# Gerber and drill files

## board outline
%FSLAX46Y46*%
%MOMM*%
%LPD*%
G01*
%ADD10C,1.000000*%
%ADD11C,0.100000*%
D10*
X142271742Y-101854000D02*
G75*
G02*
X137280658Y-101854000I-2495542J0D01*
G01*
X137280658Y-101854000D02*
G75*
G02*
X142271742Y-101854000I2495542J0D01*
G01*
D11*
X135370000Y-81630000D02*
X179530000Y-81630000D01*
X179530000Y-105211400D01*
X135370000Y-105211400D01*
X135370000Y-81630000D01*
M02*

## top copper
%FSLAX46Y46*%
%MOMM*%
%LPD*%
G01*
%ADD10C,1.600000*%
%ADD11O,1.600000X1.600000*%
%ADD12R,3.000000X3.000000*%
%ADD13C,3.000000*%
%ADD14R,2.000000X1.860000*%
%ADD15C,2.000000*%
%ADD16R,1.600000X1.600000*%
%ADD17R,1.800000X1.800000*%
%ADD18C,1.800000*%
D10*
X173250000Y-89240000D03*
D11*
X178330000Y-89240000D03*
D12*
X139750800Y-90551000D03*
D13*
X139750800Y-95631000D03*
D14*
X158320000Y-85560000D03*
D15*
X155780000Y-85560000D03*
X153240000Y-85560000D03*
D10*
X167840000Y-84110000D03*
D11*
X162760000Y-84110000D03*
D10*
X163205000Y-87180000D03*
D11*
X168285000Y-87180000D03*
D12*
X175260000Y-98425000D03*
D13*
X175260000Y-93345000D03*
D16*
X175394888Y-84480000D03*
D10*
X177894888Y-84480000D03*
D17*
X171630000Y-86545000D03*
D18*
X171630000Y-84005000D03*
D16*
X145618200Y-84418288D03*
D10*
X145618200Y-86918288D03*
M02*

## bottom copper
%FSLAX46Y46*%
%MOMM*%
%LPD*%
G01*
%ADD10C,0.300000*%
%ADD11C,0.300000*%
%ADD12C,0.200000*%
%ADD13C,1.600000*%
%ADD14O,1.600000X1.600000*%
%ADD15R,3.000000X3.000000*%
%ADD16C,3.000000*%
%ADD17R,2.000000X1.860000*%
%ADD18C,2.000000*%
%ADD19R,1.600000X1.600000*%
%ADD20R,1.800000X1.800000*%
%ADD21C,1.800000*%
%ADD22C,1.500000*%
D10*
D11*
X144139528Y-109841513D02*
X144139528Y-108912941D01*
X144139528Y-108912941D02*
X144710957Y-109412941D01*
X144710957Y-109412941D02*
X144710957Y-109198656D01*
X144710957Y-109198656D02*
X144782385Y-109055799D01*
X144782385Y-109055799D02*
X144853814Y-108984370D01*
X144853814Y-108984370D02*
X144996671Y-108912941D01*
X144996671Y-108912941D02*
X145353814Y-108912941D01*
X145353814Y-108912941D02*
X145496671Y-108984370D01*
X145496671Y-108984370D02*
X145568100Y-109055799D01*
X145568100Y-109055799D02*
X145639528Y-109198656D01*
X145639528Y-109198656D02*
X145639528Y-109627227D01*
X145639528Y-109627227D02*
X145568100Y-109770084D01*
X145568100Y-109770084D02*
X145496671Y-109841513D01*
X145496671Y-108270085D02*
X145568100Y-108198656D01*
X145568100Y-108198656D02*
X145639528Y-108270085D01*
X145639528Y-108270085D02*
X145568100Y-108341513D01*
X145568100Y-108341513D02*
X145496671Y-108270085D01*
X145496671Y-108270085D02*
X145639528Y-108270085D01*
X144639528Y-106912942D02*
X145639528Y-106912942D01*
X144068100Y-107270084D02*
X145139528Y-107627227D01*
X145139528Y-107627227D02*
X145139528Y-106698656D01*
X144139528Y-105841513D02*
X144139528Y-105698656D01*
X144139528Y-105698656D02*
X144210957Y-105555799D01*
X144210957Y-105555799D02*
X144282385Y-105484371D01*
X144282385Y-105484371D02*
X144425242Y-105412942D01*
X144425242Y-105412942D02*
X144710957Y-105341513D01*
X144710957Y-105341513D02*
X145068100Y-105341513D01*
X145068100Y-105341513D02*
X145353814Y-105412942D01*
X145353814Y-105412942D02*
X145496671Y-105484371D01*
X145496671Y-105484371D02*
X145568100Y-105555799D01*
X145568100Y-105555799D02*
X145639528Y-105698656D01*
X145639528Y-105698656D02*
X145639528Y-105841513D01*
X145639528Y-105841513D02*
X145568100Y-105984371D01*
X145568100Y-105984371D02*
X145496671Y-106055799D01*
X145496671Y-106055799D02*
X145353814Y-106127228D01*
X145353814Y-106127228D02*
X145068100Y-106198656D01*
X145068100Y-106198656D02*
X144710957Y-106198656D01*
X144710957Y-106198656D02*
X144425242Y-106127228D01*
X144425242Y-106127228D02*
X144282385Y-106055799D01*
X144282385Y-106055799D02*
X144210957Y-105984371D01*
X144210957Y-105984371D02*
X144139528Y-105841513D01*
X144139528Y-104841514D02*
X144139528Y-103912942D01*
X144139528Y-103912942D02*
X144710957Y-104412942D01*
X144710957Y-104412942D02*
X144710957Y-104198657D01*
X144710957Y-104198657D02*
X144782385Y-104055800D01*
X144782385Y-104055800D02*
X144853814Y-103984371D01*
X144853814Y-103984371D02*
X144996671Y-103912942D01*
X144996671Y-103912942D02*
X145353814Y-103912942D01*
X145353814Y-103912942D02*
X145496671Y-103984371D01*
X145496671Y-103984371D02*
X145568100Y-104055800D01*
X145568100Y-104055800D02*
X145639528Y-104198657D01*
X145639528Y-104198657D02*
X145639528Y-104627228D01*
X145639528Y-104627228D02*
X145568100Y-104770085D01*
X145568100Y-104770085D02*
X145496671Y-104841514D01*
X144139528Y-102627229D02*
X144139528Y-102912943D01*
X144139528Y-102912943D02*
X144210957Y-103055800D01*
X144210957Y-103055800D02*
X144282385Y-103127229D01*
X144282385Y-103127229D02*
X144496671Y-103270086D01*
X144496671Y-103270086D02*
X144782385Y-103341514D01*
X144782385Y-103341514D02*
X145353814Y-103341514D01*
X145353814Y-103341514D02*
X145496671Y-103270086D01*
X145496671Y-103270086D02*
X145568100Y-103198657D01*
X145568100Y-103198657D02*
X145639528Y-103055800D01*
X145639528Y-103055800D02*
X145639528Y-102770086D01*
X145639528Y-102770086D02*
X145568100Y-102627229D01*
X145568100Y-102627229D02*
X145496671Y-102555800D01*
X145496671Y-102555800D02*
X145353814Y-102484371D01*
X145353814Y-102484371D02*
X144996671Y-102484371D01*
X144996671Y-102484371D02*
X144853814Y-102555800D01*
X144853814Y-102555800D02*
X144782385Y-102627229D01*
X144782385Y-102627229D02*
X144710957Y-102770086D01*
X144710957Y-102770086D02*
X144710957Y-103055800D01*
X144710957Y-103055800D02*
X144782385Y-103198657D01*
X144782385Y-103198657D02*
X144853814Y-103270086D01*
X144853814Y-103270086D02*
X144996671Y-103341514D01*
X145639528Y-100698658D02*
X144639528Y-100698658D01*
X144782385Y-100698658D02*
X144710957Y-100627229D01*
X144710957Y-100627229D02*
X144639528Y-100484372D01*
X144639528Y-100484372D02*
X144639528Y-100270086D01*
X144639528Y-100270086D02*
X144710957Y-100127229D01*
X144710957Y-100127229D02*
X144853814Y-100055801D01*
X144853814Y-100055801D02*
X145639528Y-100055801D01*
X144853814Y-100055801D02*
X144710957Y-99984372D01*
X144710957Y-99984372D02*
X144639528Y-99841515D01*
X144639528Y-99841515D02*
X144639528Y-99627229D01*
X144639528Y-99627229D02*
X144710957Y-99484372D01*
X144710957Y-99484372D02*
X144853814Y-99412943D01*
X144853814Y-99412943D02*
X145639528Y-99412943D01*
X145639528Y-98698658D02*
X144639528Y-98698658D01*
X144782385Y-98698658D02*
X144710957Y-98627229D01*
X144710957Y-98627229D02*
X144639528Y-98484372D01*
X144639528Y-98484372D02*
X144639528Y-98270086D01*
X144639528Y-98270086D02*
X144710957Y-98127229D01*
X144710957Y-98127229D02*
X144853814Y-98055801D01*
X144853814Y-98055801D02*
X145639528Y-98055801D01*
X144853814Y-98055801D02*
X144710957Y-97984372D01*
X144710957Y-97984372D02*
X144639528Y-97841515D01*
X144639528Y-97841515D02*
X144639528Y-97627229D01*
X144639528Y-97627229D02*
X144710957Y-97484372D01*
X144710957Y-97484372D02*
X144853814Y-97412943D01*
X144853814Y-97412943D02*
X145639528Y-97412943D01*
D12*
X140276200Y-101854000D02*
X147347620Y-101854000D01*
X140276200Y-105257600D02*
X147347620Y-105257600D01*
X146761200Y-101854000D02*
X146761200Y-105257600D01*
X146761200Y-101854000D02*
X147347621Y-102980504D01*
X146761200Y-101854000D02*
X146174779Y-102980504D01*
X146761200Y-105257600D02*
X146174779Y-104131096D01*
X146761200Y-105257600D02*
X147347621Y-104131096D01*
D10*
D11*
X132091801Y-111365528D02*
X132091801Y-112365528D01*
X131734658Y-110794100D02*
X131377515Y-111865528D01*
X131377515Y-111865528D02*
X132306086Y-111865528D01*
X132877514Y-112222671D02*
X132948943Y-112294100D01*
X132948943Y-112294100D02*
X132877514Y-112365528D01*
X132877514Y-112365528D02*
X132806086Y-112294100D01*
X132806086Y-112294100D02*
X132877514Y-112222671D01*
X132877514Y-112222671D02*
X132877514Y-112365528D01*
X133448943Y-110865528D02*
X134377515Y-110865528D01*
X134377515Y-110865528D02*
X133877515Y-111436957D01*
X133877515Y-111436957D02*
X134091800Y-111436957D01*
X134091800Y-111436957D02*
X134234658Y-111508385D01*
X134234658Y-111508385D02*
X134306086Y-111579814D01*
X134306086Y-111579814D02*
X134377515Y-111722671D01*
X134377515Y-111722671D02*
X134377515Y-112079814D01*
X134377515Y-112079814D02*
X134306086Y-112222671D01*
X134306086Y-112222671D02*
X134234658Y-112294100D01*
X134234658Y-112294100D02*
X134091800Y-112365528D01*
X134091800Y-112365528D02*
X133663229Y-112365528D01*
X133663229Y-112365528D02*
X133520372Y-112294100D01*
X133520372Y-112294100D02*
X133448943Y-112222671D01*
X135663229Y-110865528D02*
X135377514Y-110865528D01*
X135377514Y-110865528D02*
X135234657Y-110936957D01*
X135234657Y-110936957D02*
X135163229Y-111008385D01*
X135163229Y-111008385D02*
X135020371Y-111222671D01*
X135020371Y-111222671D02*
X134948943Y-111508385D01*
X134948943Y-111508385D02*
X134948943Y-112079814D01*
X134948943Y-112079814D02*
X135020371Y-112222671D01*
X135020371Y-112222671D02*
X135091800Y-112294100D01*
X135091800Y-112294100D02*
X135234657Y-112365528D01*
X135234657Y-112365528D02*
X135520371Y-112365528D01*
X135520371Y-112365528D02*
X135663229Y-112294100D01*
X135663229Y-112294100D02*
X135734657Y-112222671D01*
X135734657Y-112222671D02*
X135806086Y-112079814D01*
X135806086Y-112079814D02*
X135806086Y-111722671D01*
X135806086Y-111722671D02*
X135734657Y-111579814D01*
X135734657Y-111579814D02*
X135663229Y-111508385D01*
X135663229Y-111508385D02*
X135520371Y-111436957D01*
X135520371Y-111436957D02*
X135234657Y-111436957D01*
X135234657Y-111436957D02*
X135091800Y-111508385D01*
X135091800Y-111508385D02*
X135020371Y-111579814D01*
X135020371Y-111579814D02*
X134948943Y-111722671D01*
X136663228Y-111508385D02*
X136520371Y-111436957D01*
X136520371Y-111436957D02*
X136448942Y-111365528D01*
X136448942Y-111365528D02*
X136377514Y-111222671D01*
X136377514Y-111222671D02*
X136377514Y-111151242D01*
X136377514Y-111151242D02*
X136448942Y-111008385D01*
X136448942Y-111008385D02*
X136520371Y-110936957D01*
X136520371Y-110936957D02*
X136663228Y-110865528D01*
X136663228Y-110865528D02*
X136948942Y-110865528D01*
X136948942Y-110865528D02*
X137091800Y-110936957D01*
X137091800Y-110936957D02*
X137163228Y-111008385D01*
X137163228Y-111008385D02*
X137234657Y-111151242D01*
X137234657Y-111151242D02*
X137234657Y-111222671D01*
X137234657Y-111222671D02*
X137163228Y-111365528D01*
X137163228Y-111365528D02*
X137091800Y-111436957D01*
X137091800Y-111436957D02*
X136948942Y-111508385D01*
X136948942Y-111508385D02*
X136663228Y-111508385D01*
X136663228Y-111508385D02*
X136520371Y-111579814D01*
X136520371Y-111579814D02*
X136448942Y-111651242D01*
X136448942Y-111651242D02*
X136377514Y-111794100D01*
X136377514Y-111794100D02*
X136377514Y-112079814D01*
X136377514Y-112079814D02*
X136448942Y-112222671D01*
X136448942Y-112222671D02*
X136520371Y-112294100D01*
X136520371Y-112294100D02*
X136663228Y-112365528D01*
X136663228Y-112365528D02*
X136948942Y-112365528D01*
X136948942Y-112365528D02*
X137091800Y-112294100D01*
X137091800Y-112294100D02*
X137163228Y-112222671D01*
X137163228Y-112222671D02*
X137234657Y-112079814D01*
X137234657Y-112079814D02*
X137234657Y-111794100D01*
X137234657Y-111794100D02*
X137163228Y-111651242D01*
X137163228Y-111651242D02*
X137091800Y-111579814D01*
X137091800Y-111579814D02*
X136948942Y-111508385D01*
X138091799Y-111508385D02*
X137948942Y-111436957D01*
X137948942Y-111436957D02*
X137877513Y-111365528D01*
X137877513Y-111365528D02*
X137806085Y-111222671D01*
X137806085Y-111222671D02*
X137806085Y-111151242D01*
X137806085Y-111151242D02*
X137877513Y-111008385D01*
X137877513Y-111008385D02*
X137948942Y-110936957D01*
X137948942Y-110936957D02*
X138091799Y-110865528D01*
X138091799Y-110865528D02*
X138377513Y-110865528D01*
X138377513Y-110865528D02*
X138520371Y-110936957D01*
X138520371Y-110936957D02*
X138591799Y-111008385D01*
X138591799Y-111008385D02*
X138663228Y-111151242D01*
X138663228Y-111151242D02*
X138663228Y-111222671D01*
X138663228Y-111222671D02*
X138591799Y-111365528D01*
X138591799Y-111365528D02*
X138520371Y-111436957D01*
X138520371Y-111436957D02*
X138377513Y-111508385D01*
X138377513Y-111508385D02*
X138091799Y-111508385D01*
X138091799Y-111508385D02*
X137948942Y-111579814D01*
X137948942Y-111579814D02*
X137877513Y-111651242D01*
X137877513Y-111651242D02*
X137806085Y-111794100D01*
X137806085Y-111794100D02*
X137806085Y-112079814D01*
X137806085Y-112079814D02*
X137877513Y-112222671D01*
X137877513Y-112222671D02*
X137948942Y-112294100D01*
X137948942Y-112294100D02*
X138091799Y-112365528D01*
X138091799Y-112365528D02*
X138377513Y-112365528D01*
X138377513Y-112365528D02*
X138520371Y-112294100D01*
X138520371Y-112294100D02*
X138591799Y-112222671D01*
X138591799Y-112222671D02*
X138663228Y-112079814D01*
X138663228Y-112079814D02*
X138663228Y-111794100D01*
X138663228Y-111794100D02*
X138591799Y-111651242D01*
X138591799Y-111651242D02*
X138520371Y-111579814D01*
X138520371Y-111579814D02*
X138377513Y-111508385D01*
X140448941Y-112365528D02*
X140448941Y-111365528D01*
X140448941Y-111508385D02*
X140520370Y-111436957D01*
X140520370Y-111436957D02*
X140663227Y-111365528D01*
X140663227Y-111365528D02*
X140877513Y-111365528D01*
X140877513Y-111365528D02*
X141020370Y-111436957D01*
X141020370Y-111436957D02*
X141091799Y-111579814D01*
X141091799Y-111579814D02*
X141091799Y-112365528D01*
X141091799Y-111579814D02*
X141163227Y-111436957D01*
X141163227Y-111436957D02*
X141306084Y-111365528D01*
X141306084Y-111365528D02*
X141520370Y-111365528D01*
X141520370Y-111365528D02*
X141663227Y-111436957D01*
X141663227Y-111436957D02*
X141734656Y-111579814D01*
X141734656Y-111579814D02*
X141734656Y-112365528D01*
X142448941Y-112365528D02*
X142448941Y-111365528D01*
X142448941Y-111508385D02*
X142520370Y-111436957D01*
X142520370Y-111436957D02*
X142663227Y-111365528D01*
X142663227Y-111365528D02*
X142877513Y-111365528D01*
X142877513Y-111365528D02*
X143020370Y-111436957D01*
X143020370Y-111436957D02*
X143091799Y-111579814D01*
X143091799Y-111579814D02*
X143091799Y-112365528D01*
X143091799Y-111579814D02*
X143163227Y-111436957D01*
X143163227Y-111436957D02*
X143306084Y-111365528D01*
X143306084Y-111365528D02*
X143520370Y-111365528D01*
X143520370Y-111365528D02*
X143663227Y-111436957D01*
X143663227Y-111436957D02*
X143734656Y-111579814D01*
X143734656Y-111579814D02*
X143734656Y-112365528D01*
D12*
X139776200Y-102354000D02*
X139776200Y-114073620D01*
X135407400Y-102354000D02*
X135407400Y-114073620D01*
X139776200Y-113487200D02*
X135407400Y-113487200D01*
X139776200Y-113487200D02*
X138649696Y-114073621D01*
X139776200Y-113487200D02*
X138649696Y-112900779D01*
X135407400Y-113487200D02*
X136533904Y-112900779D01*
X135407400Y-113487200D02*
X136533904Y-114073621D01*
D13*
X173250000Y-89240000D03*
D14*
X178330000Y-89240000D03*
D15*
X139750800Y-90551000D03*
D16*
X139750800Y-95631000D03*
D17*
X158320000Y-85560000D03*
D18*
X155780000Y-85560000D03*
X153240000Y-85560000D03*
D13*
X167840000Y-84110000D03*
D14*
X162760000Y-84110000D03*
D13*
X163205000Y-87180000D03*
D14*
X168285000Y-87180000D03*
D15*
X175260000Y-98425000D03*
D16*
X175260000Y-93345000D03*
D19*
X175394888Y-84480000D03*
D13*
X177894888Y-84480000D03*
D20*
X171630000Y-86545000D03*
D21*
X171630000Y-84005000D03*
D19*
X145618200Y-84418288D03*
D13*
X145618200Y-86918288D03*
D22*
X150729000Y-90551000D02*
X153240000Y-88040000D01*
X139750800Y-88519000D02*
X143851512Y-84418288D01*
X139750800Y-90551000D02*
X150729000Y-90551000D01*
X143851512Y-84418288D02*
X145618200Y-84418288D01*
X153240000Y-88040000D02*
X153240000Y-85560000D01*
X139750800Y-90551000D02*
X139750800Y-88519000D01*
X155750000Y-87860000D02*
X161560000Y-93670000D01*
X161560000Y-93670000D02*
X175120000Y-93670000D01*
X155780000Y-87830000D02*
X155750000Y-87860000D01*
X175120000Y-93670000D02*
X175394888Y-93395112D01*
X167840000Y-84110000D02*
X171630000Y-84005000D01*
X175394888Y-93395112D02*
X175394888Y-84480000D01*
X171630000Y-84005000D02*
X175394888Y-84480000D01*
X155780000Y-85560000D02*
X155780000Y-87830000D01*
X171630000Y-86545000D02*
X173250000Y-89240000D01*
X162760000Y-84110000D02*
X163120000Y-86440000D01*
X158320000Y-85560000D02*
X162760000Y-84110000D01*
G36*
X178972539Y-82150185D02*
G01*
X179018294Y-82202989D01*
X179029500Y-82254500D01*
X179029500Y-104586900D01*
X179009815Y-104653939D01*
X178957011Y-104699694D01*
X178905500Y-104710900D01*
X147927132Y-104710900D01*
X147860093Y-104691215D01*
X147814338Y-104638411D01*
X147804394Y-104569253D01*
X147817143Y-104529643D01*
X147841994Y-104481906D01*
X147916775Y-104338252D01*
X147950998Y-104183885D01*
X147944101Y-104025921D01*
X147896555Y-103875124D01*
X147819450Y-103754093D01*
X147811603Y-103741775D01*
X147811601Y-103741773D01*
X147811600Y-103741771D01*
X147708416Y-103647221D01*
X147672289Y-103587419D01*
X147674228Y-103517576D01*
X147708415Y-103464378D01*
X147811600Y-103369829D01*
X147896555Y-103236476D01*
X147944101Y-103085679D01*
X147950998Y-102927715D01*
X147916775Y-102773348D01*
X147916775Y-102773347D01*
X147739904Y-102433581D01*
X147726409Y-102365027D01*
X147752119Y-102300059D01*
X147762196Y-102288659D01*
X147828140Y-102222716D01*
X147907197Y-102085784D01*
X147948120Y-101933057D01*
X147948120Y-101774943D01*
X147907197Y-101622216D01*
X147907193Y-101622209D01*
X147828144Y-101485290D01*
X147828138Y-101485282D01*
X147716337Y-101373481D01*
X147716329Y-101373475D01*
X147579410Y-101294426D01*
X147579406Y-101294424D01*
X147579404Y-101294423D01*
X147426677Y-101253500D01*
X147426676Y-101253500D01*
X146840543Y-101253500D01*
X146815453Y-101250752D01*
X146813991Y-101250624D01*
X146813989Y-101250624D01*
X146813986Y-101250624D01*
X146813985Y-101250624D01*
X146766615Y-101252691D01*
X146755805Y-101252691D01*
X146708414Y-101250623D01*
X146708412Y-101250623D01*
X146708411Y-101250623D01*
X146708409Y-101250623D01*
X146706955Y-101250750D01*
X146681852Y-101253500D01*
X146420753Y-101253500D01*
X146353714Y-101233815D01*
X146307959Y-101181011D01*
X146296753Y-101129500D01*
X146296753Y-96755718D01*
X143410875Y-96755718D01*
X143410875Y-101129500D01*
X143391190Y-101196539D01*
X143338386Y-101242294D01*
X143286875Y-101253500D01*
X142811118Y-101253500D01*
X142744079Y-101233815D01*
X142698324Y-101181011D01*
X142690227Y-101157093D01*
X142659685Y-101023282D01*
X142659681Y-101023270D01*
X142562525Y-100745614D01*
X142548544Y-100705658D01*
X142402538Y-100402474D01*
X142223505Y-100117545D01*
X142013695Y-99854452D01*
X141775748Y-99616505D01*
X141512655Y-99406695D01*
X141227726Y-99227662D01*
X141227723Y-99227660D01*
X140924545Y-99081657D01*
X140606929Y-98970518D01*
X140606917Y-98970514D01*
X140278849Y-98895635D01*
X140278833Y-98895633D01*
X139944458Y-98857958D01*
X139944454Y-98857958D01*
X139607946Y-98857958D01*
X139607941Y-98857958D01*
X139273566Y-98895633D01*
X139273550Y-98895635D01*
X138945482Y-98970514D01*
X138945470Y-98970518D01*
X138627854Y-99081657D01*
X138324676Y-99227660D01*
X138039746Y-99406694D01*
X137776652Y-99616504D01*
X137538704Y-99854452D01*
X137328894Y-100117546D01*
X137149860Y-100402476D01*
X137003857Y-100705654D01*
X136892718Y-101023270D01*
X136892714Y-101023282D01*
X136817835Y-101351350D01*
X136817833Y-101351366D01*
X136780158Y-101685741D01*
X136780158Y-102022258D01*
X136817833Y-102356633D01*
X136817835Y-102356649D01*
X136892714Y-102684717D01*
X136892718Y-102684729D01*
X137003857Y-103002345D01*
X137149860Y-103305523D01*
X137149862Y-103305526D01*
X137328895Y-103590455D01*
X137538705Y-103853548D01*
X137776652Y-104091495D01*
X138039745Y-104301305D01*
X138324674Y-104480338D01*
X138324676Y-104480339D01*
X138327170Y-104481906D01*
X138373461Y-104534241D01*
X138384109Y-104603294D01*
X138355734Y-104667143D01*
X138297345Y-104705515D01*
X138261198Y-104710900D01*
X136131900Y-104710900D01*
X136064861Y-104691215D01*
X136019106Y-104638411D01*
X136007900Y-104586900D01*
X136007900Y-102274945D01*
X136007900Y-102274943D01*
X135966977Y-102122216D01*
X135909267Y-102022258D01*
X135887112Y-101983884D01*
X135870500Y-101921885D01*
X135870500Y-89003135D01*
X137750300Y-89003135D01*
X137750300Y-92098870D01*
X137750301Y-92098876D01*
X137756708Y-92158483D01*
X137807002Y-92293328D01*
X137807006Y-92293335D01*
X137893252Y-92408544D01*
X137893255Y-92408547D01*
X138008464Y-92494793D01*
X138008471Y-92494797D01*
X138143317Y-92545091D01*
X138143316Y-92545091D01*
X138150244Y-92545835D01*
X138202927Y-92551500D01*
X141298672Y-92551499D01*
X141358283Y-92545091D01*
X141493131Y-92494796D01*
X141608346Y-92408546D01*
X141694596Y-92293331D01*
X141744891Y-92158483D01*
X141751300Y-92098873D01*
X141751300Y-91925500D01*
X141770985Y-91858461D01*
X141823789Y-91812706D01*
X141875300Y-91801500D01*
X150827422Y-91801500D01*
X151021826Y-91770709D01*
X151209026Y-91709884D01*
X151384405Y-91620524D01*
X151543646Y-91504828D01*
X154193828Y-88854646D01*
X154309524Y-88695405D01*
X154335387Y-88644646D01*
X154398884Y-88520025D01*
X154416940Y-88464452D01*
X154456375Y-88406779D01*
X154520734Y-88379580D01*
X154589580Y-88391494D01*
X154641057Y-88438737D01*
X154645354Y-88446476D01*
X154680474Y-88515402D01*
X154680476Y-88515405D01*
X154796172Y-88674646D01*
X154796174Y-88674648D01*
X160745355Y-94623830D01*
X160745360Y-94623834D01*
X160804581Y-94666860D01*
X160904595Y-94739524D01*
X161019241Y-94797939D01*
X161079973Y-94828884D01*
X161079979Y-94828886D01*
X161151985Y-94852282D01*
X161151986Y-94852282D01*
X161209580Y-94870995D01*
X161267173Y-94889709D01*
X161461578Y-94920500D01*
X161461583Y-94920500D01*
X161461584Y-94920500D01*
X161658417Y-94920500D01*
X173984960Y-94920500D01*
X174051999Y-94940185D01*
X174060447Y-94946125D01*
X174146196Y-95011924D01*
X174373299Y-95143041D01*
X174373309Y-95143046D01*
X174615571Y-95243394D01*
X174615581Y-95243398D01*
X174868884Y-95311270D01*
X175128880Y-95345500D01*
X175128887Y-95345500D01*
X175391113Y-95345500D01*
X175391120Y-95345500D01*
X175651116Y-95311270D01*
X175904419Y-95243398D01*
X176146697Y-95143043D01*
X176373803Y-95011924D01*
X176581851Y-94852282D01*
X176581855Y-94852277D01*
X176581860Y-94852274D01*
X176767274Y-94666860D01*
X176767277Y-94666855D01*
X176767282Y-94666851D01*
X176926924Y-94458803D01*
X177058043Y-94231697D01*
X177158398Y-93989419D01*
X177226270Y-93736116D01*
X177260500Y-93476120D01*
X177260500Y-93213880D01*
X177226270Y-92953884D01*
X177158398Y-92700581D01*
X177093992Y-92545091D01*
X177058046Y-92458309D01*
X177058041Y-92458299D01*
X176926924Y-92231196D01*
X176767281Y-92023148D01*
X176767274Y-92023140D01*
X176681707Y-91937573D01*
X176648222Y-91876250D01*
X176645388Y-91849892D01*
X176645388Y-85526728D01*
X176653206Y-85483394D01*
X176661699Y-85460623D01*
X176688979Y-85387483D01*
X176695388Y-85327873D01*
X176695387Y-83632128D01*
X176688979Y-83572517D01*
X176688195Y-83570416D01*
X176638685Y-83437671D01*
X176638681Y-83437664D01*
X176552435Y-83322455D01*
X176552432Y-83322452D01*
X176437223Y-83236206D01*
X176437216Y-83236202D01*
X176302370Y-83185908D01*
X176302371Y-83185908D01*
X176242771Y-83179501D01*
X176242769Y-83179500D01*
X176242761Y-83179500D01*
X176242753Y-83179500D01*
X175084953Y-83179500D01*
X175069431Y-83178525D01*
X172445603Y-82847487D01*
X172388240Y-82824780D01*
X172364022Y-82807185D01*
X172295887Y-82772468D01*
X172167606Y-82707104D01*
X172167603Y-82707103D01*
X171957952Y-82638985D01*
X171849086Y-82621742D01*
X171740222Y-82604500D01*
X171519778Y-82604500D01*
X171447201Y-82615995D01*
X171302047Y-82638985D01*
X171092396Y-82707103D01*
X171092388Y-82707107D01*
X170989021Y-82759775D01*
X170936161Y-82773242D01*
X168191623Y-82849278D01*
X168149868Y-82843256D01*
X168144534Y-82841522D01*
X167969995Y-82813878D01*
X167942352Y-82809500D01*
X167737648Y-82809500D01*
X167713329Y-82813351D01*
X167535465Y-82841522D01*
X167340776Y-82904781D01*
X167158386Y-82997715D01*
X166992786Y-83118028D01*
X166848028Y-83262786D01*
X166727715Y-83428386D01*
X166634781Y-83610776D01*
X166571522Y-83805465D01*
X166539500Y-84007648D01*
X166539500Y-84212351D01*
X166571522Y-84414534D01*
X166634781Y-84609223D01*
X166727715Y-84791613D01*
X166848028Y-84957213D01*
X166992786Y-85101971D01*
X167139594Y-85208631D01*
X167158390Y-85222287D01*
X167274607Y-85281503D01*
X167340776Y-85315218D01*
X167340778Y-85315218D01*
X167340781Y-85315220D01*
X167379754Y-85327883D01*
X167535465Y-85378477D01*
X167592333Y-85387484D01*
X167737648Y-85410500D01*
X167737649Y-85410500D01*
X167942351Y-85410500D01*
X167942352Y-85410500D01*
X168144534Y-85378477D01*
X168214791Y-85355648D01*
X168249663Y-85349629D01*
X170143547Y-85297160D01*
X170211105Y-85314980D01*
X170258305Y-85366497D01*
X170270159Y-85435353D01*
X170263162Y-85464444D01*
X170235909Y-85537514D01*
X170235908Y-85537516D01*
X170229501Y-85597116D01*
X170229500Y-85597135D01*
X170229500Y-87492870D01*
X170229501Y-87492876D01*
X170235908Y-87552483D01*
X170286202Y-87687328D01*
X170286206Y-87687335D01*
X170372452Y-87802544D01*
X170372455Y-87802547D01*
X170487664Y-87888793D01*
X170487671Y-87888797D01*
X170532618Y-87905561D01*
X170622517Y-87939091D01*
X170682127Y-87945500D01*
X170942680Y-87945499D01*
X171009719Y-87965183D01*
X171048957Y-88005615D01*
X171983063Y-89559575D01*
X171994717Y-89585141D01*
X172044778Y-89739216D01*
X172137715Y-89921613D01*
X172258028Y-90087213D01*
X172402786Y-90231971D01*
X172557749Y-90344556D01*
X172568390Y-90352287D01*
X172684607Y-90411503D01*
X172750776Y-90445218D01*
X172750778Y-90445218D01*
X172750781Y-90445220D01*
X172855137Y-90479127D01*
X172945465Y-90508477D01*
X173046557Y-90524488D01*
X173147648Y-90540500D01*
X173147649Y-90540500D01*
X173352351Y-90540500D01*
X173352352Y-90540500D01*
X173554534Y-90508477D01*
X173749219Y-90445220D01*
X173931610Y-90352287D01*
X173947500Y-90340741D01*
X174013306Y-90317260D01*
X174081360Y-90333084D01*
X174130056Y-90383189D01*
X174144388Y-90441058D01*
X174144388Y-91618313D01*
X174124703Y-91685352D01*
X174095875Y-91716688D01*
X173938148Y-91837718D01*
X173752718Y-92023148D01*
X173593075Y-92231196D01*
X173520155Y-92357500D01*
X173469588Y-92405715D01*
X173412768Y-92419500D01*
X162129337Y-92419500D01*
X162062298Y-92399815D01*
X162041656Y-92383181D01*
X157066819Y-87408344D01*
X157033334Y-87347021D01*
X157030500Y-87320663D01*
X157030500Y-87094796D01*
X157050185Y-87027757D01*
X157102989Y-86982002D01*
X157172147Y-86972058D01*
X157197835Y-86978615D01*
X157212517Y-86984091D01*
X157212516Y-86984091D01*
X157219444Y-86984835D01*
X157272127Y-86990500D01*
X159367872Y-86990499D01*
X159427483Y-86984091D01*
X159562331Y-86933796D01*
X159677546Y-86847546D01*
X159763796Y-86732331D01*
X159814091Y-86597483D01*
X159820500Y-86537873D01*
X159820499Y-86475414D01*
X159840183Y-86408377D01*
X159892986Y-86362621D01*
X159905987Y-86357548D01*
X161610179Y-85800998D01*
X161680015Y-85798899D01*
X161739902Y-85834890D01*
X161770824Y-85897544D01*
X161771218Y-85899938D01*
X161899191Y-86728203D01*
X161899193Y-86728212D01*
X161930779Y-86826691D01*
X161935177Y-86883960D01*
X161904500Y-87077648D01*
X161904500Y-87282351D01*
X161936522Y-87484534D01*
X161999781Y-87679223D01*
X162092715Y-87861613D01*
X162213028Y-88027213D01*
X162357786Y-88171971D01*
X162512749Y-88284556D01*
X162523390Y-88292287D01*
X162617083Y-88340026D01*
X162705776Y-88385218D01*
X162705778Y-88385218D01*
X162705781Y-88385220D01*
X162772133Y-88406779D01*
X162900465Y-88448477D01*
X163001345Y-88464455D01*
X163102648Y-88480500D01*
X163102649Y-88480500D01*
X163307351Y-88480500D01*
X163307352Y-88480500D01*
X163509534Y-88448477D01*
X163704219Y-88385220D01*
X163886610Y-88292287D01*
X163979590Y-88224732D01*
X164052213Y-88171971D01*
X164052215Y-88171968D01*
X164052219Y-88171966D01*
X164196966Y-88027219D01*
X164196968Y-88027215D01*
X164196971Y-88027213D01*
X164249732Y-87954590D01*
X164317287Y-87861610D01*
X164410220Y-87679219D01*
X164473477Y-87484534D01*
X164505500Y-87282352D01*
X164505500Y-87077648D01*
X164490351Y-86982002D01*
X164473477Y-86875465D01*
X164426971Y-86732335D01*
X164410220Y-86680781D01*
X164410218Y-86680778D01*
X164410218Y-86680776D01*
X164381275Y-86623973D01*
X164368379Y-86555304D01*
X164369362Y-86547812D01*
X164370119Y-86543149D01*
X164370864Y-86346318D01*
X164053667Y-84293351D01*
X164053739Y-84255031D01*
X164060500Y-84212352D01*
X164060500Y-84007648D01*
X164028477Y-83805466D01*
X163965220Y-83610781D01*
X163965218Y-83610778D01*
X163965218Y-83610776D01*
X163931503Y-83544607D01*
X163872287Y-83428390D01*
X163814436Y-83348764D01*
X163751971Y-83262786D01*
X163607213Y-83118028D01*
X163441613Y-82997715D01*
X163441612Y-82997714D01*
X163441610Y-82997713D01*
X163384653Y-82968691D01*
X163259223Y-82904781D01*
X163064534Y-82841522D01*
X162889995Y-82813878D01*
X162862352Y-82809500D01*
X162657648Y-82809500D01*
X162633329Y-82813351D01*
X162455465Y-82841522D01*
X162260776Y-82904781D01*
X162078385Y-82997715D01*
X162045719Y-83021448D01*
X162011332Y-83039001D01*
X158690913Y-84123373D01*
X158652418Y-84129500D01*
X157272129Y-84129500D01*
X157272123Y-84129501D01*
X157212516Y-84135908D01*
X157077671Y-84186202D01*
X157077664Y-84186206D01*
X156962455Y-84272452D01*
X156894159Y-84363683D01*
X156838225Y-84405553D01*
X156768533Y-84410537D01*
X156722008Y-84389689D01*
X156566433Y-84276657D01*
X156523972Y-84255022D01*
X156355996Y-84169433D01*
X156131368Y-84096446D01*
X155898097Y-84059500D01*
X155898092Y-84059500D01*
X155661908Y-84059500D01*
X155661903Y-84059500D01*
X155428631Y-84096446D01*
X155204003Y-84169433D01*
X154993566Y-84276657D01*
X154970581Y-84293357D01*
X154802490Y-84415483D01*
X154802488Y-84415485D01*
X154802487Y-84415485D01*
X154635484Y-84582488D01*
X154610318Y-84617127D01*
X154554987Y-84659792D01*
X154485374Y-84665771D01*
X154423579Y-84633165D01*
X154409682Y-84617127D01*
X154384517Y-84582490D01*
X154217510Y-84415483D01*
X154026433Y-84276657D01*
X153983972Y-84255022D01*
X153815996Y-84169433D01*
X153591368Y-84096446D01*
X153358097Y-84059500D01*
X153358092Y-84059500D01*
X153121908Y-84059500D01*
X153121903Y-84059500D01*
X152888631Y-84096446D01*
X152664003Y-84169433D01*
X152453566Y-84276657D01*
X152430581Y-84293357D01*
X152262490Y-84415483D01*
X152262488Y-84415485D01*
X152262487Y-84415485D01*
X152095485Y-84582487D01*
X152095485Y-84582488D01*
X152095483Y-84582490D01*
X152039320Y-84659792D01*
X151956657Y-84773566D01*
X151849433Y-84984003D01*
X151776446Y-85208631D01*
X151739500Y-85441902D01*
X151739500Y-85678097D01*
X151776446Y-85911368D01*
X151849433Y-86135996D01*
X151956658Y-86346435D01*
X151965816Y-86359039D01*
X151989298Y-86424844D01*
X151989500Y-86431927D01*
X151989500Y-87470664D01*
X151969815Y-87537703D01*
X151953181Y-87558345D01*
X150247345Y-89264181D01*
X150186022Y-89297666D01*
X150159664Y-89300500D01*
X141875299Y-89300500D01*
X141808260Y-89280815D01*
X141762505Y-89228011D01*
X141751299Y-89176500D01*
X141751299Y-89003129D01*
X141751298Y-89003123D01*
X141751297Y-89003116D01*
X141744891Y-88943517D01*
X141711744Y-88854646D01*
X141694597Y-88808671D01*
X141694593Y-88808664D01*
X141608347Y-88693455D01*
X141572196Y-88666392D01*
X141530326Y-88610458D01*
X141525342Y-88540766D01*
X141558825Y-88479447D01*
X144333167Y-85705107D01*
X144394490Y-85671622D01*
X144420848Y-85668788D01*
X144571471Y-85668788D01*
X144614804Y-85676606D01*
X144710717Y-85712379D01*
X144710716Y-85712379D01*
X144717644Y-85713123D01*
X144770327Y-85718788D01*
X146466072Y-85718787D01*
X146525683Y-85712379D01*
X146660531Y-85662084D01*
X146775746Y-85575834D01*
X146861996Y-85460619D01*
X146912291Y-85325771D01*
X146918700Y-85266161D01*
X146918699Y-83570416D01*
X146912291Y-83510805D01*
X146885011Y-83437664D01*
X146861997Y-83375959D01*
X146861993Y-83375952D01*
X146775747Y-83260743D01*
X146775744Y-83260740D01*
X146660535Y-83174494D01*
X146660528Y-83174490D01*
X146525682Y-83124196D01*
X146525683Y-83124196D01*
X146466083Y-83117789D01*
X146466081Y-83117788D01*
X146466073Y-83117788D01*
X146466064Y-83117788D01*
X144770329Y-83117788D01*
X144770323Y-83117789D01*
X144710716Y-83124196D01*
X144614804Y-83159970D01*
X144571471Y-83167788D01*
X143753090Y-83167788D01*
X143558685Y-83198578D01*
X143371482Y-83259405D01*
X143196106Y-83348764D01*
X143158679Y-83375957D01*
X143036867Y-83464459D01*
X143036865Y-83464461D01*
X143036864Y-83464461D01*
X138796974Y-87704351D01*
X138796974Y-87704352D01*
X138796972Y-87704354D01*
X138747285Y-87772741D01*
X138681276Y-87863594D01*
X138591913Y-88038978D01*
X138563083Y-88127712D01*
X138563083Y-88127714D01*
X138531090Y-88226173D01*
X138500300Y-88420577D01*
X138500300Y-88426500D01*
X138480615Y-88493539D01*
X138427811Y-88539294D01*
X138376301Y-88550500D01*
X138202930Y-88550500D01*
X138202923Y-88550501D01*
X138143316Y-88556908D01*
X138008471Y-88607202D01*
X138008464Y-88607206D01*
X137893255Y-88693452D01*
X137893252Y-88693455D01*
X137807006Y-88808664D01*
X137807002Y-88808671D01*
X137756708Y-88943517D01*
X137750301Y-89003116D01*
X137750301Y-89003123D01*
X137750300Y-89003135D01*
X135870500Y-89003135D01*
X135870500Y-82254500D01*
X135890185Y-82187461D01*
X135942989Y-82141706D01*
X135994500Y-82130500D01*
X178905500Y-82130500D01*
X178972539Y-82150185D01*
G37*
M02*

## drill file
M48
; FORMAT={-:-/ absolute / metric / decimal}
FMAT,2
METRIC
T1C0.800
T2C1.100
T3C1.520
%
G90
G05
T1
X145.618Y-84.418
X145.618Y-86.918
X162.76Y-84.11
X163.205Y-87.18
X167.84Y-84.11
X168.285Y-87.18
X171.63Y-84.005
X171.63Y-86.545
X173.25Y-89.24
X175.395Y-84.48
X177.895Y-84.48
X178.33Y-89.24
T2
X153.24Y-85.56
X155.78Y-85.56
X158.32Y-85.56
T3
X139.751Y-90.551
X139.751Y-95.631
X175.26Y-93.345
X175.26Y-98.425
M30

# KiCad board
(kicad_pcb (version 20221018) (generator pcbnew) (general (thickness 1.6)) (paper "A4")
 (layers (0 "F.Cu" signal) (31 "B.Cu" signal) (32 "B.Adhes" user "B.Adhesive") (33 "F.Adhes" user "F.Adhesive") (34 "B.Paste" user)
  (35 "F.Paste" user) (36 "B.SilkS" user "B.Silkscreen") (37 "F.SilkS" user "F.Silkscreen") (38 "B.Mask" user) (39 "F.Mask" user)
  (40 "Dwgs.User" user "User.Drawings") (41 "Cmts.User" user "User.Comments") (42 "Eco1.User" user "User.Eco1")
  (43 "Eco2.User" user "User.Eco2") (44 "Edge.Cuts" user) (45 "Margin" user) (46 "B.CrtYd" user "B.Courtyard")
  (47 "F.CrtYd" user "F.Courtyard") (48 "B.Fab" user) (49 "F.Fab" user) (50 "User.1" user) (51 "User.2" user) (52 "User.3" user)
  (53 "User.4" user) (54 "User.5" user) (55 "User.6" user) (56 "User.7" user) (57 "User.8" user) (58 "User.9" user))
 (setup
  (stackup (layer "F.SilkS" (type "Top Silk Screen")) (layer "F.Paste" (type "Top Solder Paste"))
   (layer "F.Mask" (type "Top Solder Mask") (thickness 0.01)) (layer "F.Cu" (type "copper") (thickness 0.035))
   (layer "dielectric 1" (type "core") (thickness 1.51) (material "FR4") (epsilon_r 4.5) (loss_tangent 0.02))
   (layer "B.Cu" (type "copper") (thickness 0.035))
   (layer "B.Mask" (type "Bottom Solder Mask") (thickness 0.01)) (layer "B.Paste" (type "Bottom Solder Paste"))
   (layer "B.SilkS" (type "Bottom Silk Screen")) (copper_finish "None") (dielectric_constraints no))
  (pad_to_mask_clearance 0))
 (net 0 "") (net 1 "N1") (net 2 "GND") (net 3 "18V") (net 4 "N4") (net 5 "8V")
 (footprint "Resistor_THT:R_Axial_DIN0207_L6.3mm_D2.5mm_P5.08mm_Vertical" (layer "F.Cu") (at 173.25 89.24)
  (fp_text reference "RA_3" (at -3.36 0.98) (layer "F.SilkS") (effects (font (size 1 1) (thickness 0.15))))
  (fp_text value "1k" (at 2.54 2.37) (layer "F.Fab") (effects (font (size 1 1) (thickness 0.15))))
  (pad "1" thru_hole circle (at 0 0) (size 1.6 1.6) (drill 0.8) (layers "*.Cu" "*.Mask") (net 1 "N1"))
  (pad "2" thru_hole oval (at 5.08 0) (size 1.6 1.6) (drill 0.8) (layers "*.Cu" "*.Mask") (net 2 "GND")))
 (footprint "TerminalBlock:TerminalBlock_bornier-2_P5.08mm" (layer "F.Cu") (at 139.7508 90.551 -90)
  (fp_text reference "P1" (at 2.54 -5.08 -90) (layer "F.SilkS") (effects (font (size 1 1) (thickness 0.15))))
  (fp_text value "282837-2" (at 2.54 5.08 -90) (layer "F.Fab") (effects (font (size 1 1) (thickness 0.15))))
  (pad "1" thru_hole rect (at 0 0 270) (size 3 3) (drill 1.52) (layers "*.Cu" "*.Mask") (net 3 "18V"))
  (pad "2" thru_hole circle (at 5.08 0 270) (size 3 3) (drill 1.52) (layers "*.Cu" "*.Mask") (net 2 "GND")))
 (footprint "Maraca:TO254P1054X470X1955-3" (layer "F.Cu") (at 155.78 85.56 180)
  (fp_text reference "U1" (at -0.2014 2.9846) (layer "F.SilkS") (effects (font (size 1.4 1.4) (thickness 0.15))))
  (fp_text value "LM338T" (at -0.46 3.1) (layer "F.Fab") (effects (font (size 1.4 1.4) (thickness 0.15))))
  (pad "1" thru_hole rect (at -2.54 0 180) (size 2 1.86) (drill 1.1) (layers "*.Cu" "*.Mask") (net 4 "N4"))
  (pad "2" thru_hole circle (at 0 0 180) (size 2 2) (drill 1.1) (layers "*.Cu" "*.Mask") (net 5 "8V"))
  (pad "3" thru_hole circle (at 2.54 0 180) (size 2 2) (drill 1.1) (layers "*.Cu" "*.Mask") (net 3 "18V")))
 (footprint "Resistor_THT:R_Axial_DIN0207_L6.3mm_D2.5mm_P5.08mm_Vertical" (layer "F.Cu") (at 167.84 84.11 180)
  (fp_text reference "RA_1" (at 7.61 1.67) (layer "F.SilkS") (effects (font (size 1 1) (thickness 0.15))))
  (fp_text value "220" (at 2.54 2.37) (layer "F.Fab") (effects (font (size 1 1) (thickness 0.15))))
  (pad "1" thru_hole circle (at 0 0 180) (size 1.6 1.6) (drill 0.8) (layers "*.Cu" "*.Mask") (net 5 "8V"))
  (pad "2" thru_hole oval (at 5.08 0 180) (size 1.6 1.6) (drill 0.8) (layers "*.Cu" "*.Mask") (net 4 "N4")))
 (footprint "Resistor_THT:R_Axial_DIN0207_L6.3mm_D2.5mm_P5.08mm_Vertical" (layer "F.Cu") (at 163.205 87.18)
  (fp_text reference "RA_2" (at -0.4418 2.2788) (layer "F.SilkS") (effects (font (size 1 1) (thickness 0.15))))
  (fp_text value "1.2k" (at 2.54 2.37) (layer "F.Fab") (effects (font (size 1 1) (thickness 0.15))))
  (pad "1" thru_hole circle (at 0 0) (size 1.6 1.6) (drill 0.8) (layers "*.Cu" "*.Mask") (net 4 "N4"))
  (pad "2" thru_hole oval (at 5.08 0) (size 1.6 1.6) (drill 0.8) (layers "*.Cu" "*.Mask") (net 2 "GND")))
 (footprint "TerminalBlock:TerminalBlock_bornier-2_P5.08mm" (layer "F.Cu") (at 175.26 98.425 90)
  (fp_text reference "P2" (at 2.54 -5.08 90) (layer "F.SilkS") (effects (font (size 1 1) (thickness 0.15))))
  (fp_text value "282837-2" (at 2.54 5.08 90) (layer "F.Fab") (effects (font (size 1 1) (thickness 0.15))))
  (pad "1" thru_hole rect (at 0 0 90) (size 3 3) (drill 1.52) (layers "*.Cu" "*.Mask") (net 2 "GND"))
  (pad "2" thru_hole circle (at 5.08 0 90) (size 3 3) (drill 1.52) (layers "*.Cu" "*.Mask") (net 5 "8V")))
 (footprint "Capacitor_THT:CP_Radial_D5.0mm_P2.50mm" (layer "F.Cu") (at 175.394888 84.48)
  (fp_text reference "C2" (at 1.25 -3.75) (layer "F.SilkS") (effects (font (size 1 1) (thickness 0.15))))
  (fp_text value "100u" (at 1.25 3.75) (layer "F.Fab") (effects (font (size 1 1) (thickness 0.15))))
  (pad "1" thru_hole rect (at 0 0) (size 1.6 1.6) (drill 0.8) (layers "*.Cu" "*.Mask") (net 5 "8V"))
  (pad "2" thru_hole circle (at 2.5 0) (size 1.6 1.6) (drill 0.8) (layers "*.Cu" "*.Mask") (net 2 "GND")))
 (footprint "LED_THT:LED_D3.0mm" (layer "F.Cu") (at 171.63 86.545 90)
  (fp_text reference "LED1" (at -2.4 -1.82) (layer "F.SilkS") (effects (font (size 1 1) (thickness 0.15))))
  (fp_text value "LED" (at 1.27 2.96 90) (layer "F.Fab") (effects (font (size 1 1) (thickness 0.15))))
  (pad "1" thru_hole rect (at 0 0 90) (size 1.8 1.8) (drill 0.8) (layers "*.Cu" "*.Mask") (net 1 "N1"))
  (pad "2" thru_hole circle (at 2.54 0 90) (size 1.8 1.8) (drill 0.8) (layers "*.Cu" "*.Mask") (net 5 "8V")))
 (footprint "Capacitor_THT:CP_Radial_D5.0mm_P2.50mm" (layer "F.Cu") (at 145.6182 84.418288 -90)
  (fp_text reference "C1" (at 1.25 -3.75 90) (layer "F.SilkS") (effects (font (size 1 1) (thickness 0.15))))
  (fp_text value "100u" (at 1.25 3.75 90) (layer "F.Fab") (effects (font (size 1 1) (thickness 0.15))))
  (pad "1" thru_hole rect (at 0 0 270) (size 1.6 1.6) (drill 0.8) (layers "*.Cu" "*.Mask") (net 3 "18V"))
  (pad "2" thru_hole circle (at 2.5 0 270) (size 1.6 1.6) (drill 0.8) (layers "*.Cu" "*.Mask") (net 2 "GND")))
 (gr_circle (center 139.7762 101.854) (end 142.271742 101.854) (stroke (width 1) (type solid)) (fill none) (layer "Edge.Cuts"))
 (gr_rect (start 135.37 81.63) (end 179.53 105.2114) (stroke (width 0.1) (type default)) (fill none) (layer "Edge.Cuts"))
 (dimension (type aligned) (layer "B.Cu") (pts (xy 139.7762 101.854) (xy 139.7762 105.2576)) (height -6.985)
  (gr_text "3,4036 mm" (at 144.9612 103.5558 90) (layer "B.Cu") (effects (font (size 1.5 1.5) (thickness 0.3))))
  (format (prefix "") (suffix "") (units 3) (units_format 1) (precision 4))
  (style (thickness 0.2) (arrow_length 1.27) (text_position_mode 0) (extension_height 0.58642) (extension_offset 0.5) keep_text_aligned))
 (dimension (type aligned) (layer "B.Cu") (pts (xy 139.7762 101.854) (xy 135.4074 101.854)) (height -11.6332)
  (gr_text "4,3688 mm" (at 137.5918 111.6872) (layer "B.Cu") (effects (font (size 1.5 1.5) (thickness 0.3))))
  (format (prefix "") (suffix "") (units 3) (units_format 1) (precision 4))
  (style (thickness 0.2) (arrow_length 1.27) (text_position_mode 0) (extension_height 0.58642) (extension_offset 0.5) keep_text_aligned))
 (segment (start 150.729 90.551) (end 153.24 88.04) (width 1.5) (layer "B.Cu") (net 3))
 (segment (start 139.7508 88.519) (end 143.851512 84.418288) (width 1.5) (layer "B.Cu") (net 3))
 (segment (start 139.7508 90.551) (end 150.729 90.551) (width 1.5) (layer "B.Cu") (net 3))
 (segment (start 143.851512 84.418288) (end 145.6182 84.418288) (width 1.5) (layer "B.Cu") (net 3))
 (segment (start 153.24 88.04) (end 153.24 85.56) (width 1.5) (layer "B.Cu") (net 3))
 (segment (start 139.7508 90.551) (end 139.7508 88.519) (width 1.5) (layer "B.Cu") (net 3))
 (segment (start 155.75 87.86) (end 161.56 93.67) (width 1.5) (layer "B.Cu") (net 5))
 (segment (start 161.56 93.67) (end 175.12 93.67) (width 1.5) (layer "B.Cu") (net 5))
 (segment (start 155.78 87.83) (end 155.75 87.86) (width 1.5) (layer "B.Cu") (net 5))
 (segment (start 175.12 93.67) (end 175.394888 93.395112) (width 1.5) (layer "B.Cu") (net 5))
 (segment (start 167.84 84.11) (end 171.63 84.005) (width 1.5) (layer "B.Cu") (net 5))
 (segment (start 175.394888 93.395112) (end 175.394888 84.48) (width 1.5) (layer "B.Cu") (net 5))
 (segment (start 171.63 84.005) (end 175.394888 84.48) (width 1.5) (layer "B.Cu") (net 5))
 (segment (start 155.78 85.56) (end 155.78 87.83) (width 1.5) (layer "B.Cu") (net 5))
 (segment (start 171.63 86.545) (end 173.25 89.24) (width 1.5) (layer "B.Cu") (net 1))
 (segment (start 162.76 84.11) (end 163.12 86.44) (width 1.5) (layer "B.Cu") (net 4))
 (segment (start 158.32 85.56) (end 162.76 84.11) (width 1.5) (layer "B.Cu") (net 4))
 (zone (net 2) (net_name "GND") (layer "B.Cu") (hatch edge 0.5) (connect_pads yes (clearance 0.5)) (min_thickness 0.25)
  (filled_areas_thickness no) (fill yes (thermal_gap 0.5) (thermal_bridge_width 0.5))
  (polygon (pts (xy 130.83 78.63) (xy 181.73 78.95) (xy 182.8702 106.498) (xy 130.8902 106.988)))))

